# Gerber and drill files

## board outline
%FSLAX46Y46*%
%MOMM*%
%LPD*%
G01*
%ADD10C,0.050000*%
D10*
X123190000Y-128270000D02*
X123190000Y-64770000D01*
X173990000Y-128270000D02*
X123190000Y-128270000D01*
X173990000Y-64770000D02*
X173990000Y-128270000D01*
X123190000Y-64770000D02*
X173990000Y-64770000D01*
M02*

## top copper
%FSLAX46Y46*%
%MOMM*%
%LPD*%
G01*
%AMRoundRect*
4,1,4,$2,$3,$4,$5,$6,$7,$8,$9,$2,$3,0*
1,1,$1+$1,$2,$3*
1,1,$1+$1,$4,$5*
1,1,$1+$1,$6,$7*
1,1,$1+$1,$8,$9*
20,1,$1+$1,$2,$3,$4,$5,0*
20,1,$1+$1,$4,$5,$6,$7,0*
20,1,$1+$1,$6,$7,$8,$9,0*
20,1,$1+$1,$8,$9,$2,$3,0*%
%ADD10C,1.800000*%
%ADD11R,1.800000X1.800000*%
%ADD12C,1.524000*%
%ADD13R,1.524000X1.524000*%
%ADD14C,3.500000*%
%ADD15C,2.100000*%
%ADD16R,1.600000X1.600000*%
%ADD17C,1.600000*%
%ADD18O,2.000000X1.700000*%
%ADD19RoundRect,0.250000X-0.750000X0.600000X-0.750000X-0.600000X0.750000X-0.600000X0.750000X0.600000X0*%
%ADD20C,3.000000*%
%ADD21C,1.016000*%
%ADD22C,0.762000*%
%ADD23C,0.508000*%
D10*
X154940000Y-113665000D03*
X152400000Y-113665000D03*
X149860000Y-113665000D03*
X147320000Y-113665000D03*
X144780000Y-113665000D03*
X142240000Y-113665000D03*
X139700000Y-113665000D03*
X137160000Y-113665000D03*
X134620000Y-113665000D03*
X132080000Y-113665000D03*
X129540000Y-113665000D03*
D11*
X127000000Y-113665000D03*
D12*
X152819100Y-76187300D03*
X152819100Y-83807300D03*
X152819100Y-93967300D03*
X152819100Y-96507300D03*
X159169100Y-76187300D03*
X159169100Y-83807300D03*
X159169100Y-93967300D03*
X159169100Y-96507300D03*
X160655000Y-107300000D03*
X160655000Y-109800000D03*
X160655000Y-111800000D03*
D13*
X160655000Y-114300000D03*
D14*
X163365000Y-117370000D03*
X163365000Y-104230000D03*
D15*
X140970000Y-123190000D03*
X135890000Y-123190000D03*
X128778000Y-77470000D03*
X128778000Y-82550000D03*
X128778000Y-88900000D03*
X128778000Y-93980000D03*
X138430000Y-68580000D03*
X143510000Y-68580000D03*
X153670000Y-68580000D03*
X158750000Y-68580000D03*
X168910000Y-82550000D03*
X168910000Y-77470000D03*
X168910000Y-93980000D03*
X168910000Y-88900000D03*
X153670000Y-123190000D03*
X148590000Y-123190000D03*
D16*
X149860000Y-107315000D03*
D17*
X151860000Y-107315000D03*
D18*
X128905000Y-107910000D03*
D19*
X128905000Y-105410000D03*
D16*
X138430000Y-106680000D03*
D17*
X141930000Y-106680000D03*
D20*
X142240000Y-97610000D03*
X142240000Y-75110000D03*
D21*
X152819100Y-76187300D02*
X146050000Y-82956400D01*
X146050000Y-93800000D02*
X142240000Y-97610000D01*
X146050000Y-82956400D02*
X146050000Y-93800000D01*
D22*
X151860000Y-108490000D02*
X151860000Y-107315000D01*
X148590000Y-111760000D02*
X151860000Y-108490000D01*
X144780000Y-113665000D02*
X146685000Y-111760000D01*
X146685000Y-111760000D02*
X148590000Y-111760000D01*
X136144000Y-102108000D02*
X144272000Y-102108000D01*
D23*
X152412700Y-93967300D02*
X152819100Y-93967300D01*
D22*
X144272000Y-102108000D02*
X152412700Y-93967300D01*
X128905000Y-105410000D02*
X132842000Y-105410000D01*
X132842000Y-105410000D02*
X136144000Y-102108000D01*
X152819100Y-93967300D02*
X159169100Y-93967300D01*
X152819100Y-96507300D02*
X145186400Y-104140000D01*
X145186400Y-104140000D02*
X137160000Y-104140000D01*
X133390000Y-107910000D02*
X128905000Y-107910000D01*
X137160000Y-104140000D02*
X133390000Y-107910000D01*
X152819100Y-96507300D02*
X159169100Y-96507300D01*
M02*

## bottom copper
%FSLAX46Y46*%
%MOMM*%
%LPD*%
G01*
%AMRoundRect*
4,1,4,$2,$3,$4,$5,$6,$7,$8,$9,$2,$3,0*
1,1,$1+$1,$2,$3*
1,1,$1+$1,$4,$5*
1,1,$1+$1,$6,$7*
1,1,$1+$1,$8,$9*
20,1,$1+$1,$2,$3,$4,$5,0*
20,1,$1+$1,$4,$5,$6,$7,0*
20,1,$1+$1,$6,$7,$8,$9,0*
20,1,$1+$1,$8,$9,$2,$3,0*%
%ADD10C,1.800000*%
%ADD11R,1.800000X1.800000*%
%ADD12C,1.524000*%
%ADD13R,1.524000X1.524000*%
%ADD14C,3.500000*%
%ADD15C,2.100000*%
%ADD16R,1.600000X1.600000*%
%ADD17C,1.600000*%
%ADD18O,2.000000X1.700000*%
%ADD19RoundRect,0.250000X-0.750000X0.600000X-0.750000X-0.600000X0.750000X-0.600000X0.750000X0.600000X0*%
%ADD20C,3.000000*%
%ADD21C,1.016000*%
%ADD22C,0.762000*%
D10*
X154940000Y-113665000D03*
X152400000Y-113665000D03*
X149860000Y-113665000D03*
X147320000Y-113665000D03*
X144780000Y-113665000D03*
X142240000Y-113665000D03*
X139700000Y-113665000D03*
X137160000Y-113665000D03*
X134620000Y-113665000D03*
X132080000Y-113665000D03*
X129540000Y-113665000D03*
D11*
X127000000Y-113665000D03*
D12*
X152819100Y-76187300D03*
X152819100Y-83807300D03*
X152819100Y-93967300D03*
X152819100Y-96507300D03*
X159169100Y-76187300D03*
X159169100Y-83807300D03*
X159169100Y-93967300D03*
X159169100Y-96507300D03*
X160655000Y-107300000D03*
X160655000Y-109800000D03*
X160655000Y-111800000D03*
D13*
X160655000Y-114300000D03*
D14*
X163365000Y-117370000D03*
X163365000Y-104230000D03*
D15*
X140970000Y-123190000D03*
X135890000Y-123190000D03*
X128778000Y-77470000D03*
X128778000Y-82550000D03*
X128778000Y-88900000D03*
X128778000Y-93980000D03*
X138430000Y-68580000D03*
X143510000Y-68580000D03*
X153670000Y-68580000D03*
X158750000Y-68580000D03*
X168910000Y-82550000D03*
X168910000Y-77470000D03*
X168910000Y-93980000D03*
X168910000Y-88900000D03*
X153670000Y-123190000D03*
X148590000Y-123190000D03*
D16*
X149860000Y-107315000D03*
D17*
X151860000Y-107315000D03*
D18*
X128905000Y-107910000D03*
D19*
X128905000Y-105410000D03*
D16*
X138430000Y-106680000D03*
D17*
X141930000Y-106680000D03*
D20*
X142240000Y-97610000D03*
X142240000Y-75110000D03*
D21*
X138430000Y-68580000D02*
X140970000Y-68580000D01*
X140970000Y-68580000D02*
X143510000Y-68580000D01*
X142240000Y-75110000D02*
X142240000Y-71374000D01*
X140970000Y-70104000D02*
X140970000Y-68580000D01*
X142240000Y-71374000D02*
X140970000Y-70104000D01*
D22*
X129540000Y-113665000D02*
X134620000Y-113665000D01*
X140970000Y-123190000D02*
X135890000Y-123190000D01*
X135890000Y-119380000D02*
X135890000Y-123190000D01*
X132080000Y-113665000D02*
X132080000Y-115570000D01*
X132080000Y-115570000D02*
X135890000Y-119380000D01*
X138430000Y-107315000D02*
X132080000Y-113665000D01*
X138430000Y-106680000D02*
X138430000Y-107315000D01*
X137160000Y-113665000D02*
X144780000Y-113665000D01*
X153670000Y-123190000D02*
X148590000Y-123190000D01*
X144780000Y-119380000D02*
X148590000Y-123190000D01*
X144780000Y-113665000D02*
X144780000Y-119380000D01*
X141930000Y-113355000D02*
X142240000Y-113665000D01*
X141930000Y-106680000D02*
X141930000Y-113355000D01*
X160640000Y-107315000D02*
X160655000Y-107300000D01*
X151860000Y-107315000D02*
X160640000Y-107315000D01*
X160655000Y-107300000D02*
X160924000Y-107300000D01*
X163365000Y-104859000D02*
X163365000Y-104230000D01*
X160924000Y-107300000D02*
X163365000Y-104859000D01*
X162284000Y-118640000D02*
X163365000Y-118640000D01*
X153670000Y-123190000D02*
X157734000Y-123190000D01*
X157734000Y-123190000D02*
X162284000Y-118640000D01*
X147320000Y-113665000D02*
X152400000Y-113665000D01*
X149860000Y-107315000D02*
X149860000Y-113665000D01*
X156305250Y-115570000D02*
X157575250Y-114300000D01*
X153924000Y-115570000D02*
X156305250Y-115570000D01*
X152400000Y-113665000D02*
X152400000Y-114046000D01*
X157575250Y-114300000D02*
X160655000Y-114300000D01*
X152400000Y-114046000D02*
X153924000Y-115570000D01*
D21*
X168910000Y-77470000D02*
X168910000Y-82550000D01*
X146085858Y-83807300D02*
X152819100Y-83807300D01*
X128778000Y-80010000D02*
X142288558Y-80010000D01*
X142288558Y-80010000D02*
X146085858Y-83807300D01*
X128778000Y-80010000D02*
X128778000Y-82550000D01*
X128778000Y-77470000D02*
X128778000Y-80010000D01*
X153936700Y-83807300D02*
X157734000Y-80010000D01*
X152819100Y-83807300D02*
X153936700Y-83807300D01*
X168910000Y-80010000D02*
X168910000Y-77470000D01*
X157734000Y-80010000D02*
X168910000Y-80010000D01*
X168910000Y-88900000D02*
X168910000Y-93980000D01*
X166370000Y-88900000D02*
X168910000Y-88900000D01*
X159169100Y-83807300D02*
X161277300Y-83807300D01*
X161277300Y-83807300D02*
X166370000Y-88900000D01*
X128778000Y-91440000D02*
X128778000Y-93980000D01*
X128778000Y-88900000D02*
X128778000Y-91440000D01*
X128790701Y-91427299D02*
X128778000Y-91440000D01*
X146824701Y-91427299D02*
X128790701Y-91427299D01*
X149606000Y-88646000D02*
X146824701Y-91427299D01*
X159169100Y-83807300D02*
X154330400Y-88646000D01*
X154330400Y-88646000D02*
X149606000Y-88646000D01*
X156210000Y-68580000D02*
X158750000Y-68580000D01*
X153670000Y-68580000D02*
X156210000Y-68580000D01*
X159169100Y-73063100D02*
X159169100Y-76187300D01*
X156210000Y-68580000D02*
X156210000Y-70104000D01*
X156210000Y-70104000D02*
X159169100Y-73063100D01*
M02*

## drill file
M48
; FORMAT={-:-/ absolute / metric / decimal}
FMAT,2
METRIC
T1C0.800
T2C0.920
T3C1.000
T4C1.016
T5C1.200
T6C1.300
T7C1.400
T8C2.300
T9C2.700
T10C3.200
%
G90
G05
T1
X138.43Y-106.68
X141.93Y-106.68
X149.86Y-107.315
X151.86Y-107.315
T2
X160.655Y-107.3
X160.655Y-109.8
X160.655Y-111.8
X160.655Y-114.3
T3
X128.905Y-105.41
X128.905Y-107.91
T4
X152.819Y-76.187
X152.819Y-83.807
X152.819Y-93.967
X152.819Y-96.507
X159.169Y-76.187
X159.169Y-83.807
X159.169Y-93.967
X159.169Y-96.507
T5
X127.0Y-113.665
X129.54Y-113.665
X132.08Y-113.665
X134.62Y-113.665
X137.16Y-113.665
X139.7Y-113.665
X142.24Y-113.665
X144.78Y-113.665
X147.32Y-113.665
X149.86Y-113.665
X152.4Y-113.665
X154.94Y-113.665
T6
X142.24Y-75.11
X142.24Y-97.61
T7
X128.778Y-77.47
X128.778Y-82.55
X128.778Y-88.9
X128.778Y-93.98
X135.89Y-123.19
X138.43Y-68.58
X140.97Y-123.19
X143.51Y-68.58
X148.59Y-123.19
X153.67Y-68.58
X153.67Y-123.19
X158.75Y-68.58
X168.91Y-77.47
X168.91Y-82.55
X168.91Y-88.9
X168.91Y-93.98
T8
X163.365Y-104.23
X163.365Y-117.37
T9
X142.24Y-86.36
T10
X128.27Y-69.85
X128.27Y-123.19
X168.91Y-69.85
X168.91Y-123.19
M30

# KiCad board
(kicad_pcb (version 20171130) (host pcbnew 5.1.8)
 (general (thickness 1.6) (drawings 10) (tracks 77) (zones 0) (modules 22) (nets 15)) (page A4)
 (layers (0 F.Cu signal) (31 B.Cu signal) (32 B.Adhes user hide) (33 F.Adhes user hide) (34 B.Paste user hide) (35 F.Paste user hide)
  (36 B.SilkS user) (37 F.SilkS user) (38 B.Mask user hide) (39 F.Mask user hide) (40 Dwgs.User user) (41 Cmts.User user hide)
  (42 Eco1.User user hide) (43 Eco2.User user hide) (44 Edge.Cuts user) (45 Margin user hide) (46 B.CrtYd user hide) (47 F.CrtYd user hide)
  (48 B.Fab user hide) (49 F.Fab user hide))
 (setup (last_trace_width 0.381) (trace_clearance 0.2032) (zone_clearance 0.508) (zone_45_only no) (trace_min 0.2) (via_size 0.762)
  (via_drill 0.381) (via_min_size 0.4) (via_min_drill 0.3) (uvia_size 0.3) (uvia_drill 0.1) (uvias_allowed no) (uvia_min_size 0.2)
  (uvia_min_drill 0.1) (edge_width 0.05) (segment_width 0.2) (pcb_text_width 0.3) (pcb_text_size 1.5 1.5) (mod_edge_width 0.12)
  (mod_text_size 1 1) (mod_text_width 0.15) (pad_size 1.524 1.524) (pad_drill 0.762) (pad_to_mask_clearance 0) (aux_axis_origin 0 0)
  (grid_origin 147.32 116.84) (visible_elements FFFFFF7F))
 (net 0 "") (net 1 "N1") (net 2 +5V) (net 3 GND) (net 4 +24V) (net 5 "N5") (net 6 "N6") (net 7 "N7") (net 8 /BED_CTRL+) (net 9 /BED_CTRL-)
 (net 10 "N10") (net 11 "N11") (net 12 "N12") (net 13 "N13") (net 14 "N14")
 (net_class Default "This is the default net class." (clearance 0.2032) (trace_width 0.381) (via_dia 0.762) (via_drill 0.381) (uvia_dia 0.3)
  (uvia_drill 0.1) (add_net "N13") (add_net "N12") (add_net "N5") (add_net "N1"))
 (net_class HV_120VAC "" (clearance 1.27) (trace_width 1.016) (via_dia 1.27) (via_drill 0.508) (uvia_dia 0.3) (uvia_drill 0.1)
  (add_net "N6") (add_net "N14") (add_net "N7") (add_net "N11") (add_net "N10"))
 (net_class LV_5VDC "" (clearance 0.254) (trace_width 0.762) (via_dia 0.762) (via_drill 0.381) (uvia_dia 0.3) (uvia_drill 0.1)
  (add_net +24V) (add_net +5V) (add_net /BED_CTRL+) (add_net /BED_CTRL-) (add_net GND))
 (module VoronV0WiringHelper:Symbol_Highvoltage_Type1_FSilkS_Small (layer F.Cu) (at 131.064 71.628)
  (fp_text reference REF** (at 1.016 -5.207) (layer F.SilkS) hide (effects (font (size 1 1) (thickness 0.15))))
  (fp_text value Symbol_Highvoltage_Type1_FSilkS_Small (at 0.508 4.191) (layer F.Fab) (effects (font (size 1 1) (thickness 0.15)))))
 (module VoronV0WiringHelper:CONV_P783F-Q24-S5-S (layer F.Cu) (at 127 113.665)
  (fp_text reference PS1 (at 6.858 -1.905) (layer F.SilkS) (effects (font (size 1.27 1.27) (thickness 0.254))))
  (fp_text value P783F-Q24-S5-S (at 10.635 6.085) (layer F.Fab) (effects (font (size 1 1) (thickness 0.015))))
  (pad 12 thru_hole circle (at 27.94 0) (size 1.8 1.8) (drill 1.2) (layers *.Cu *.Mask) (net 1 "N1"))
  (pad 11 thru_hole circle (at 25.4 0) (size 1.8 1.8) (drill 1.2) (layers *.Cu *.Mask) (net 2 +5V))
  (pad 10 thru_hole circle (at 22.86 0) (size 1.8 1.8) (drill 1.2) (layers *.Cu *.Mask) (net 2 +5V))
  (pad 9 thru_hole circle (at 20.32 0) (size 1.8 1.8) (drill 1.2) (layers *.Cu *.Mask) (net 2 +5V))
  (pad 8 thru_hole circle (at 17.78 0) (size 1.8 1.8) (drill 1.2) (layers *.Cu *.Mask) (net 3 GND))
  (pad 7 thru_hole circle (at 15.24 0) (size 1.8 1.8) (drill 1.2) (layers *.Cu *.Mask) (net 3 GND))
  (pad 6 thru_hole circle (at 12.7 0) (size 1.8 1.8) (drill 1.2) (layers *.Cu *.Mask) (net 3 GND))
  (pad 5 thru_hole circle (at 10.16 0) (size 1.8 1.8) (drill 1.2) (layers *.Cu *.Mask) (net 3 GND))
  (pad 4 thru_hole circle (at 7.62 0) (size 1.8 1.8) (drill 1.2) (layers *.Cu *.Mask) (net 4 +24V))
  (pad 3 thru_hole circle (at 5.08 0) (size 1.8 1.8) (drill 1.2) (layers *.Cu *.Mask) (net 4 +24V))
  (pad 2 thru_hole circle (at 2.54 0) (size 1.8 1.8) (drill 1.2) (layers *.Cu *.Mask) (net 4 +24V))
  (pad 1 thru_hole rect (at 0 0) (size 1.8 1.8) (drill 1.2) (layers *.Cu *.Mask) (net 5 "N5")))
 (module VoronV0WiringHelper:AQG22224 (layer F.Cu) (at 151.765 86.36 180)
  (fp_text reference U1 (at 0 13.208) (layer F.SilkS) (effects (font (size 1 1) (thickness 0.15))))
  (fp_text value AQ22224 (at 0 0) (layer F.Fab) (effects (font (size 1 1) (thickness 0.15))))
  (pad 4 thru_hole circle (at -1.0541 10.1727 180) (size 1.524 1.524) (drill 1.016) (layers *.Cu *.Mask) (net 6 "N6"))
  (pad 3 thru_hole circle (at -1.0541 2.5527 180) (size 1.524 1.524) (drill 1.016) (layers *.Cu *.Mask) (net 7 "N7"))
  (pad 2 thru_hole circle (at -1.0541 -7.6073 180) (size 1.524 1.524) (drill 1.016) (layers *.Cu *.Mask) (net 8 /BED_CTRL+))
  (pad 1 thru_hole circle (at -1.0541 -10.1473 180) (size 1.524 1.524) (drill 1.016) (layers *.Cu *.Mask) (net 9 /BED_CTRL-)))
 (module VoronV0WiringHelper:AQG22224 (layer F.Cu) (at 158.115 86.36 180)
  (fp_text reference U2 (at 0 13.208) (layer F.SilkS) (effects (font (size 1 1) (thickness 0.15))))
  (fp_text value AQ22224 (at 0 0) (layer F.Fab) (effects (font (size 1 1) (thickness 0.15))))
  (pad 4 thru_hole circle (at -1.0541 10.1727 180) (size 1.524 1.524) (drill 1.016) (layers *.Cu *.Mask) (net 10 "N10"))
  (pad 3 thru_hole circle (at -1.0541 2.5527 180) (size 1.524 1.524) (drill 1.016) (layers *.Cu *.Mask) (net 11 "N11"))
  (pad 2 thru_hole circle (at -1.0541 -7.6073 180) (size 1.524 1.524) (drill 1.016) (layers *.Cu *.Mask) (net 8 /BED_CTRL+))
  (pad 1 thru_hole circle (at -1.0541 -10.1473 180) (size 1.524 1.524) (drill 1.016) (layers *.Cu *.Mask) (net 9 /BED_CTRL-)))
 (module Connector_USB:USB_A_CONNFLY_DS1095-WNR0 (layer F.Cu) (at 160.655 114.3 90)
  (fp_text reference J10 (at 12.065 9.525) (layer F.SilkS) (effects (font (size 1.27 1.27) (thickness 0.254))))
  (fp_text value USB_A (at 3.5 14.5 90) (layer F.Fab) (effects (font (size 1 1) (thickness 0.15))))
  (pad 4 thru_hole circle (at 7 0 90) (size 1.524 1.524) (drill 0.92) (layers *.Cu *.Mask) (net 3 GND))
  (pad 3 thru_hole circle (at 4.5 0 90) (size 1.524 1.524) (drill 0.92) (layers *.Cu *.Mask) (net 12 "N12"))
  (pad 2 thru_hole circle (at 2.5 0 90) (size 1.524 1.524) (drill 0.92) (layers *.Cu *.Mask) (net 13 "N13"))
  (pad 1 thru_hole rect (at 0 0 90) (size 1.524 1.524) (drill 0.92) (layers *.Cu *.Mask) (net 2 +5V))
  (pad 5 thru_hole circle (at -3.07 2.71 90) (size 3.5 3.5) (drill 2.3) (layers *.Cu *.Mask) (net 3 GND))
  (pad 5 thru_hole circle (at 10.07 2.71 90) (size 3.5 3.5) (drill 2.3) (layers *.Cu *.Mask) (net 3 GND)))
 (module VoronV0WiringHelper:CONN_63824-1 (layer F.Cu) (at 138.43 123.19 180)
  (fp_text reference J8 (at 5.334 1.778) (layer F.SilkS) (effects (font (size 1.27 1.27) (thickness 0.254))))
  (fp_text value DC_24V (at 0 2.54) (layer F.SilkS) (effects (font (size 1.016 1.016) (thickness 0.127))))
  (pad 1 thru_hole circle (at -2.54 0 180) (size 2.1 2.1) (drill 1.4) (layers *.Cu *.Mask) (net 4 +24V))
  (pad 1 thru_hole circle (at 2.54 0 180) (size 2.1 2.1) (drill 1.4) (layers *.Cu *.Mask) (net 4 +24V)))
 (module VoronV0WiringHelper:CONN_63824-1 (layer F.Cu) (at 128.778 80.01 270)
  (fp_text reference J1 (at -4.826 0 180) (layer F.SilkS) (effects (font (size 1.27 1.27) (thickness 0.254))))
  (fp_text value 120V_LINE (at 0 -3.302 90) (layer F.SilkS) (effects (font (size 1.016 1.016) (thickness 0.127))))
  (pad 1 thru_hole circle (at -2.54 0 270) (size 2.1 2.1) (drill 1.4) (layers *.Cu *.Mask) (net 7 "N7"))
  (pad 1 thru_hole circle (at 2.54 0 270) (size 2.1 2.1) (drill 1.4) (layers *.Cu *.Mask) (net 7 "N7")))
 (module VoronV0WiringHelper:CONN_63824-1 (layer F.Cu) (at 128.778 91.44 270)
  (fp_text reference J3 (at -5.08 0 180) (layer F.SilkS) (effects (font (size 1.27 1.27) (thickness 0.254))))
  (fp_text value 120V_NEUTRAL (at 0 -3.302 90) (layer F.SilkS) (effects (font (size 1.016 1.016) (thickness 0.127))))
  (pad 1 thru_hole circle (at -2.54 0 270) (size 2.1 2.1) (drill 1.4) (layers *.Cu *.Mask) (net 11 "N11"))
  (pad 1 thru_hole circle (at 2.54 0 270) (size 2.1 2.1) (drill 1.4) (layers *.Cu *.Mask) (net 11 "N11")))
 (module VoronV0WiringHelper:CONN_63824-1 (layer F.Cu) (at 140.97 68.58)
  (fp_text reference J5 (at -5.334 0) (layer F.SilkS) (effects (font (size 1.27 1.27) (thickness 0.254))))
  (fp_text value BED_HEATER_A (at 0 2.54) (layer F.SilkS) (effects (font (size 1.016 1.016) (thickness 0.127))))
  (pad 1 thru_hole circle (at -2.54 0) (size 2.1 2.1) (drill 1.4) (layers *.Cu *.Mask) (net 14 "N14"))
  (pad 1 thru_hole circle (at 2.54 0) (size 2.1 2.1) (drill 1.4) (layers *.Cu *.Mask) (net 14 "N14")))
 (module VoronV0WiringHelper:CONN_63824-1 (layer F.Cu) (at 156.21 68.58)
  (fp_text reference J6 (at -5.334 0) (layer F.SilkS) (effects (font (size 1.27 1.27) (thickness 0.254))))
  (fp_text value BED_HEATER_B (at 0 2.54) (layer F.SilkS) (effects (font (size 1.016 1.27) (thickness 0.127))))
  (pad 1 thru_hole circle (at -2.54 0) (size 2.1 2.1) (drill 1.4) (layers *.Cu *.Mask) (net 10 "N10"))
  (pad 1 thru_hole circle (at 2.54 0) (size 2.1 2.1) (drill 1.4) (layers *.Cu *.Mask) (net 10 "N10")))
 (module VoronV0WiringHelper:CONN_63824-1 (layer F.Cu) (at 168.91 80.01 90)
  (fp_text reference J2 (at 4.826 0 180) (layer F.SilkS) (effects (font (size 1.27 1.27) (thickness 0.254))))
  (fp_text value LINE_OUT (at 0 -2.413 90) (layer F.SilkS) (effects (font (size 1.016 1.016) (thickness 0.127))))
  (pad 1 thru_hole circle (at -2.54 0 90) (size 2.1 2.1) (drill 1.4) (layers *.Cu *.Mask) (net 7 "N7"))
  (pad 1 thru_hole circle (at 2.54 0 90) (size 2.1 2.1) (drill 1.4) (layers *.Cu *.Mask) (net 7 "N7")))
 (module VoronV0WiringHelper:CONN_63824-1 (layer F.Cu) (at 168.91 91.44 90)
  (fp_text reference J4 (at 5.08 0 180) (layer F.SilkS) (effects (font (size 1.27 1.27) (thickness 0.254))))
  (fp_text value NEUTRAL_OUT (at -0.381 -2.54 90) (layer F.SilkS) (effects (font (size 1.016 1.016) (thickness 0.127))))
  (pad 1 thru_hole circle (at -2.54 0 90) (size 2.1 2.1) (drill 1.4) (layers *.Cu *.Mask) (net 11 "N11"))
  (pad 1 thru_hole circle (at 2.54 0 90) (size 2.1 2.1) (drill 1.4) (layers *.Cu *.Mask) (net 11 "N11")))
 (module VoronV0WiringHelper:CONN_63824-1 (layer F.Cu) (at 151.13 123.19 180)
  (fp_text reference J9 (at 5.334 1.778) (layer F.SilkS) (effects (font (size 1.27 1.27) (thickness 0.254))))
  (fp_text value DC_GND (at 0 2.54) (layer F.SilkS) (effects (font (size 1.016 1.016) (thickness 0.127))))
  (pad 1 thru_hole circle (at -2.54 0 180) (size 2.1 2.1) (drill 1.4) (layers *.Cu *.Mask) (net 3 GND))
  (pad 1 thru_hole circle (at 2.54 0 180) (size 2.1 2.1) (drill 1.4) (layers *.Cu *.Mask) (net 3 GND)))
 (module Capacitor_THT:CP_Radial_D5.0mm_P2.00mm (layer F.Cu) (at 149.86 107.315)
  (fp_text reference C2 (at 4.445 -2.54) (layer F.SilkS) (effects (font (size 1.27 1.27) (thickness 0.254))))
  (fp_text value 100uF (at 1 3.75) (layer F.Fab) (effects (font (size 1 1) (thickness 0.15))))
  (pad 1 thru_hole rect (at 0 0) (size 1.6 1.6) (drill 0.8) (layers *.Cu *.Mask) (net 2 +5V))
  (pad 2 thru_hole circle (at 2 0) (size 1.6 1.6) (drill 0.8) (layers *.Cu *.Mask) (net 3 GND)))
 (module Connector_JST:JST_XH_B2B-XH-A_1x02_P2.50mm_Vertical (layer F.Cu) (at 128.905 105.41 270)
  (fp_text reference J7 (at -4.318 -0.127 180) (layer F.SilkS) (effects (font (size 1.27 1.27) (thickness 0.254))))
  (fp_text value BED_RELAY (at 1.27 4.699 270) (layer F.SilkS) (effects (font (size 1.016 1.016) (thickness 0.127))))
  (pad 2 thru_hole oval (at 2.5 0 270) (size 1.7 2) (drill 1) (layers *.Cu *.Mask) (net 9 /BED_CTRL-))
  (pad 1 thru_hole roundrect (at 0 0 270) (size 1.7 2) (drill 1) (layers *.Cu *.Mask) (roundrect_rratio 0.1470588235294118)
   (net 8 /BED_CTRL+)))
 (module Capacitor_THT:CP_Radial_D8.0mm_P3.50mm (layer F.Cu) (at 138.43 106.68)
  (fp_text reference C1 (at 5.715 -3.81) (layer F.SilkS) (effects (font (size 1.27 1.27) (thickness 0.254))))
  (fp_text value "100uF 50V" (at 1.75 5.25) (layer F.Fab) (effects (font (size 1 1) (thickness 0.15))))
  (pad 1 thru_hole rect (at 0 0) (size 1.6 1.6) (drill 0.8) (layers *.Cu *.Mask) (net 4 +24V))
  (pad 2 thru_hole circle (at 3.5 0) (size 1.6 1.6) (drill 0.8) (layers *.Cu *.Mask) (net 3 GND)))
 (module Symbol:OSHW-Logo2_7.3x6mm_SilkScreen (layer F.Cu) (at 161.29 123.825)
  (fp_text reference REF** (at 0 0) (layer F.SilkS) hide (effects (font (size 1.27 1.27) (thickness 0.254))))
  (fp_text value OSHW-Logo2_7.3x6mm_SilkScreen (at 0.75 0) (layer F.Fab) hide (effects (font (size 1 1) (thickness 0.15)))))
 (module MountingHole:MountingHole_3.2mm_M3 (layer F.Cu) (at 168.91 123.19)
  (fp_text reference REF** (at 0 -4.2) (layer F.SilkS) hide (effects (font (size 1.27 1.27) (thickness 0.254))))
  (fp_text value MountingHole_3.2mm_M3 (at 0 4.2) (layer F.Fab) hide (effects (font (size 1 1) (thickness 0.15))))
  (pad 1 np_thru_hole circle (at 0 0) (size 3.2 3.2) (drill 3.2) (layers *.Cu *.Mask)))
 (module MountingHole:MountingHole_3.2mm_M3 (layer F.Cu) (at 168.91 69.85)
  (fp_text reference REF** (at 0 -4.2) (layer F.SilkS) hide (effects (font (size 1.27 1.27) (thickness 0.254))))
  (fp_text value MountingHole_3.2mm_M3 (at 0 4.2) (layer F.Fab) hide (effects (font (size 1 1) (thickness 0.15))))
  (pad 1 np_thru_hole circle (at 0 0) (size 3.2 3.2) (drill 3.2) (layers *.Cu *.Mask)))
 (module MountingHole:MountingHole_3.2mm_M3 (layer F.Cu) (at 128.27 69.85)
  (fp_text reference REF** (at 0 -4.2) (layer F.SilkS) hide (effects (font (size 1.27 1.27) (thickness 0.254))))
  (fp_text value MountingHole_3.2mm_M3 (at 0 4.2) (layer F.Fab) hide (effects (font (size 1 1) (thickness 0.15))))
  (pad 1 np_thru_hole circle (at 0 0) (size 3.2 3.2) (drill 3.2) (layers *.Cu *.Mask)))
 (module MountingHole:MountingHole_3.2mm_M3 (layer F.Cu) (at 128.27 123.19)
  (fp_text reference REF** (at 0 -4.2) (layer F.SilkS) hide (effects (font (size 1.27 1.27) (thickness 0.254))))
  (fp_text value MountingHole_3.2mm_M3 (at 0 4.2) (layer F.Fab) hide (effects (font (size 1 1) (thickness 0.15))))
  (pad 1 np_thru_hole circle (at 0 0) (size 3.2 3.2) (drill 3.2) (layers *.Cu *.Mask)))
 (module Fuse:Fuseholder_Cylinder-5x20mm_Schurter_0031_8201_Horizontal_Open (layer F.Cu) (at 142.24 97.61 90)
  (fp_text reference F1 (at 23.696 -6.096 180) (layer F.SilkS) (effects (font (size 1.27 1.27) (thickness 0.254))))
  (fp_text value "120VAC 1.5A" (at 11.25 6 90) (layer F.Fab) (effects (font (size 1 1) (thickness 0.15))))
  (pad 1 thru_hole circle (at 0 0 90) (size 3 3) (drill 1.3) (layers *.Cu *.Mask) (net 6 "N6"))
  (pad 2 thru_hole circle (at 22.5 0 90) (size 3 3) (drill 1.3) (layers *.Cu *.Mask) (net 14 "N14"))
  (pad "" np_thru_hole circle (at 11.25 0 90) (size 2.7 2.7) (drill 2.7) (layers *.Cu *.Mask)))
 (gr_line (start 123.19 128.27) (end 123.19 64.77) (layer Edge.Cuts) (width 0.05))
 (gr_line (start 173.99 128.27) (end 123.19 128.27) (layer Edge.Cuts) (width 0.05))
 (gr_line (start 173.99 64.77) (end 173.99 128.27) (layer Edge.Cuts) (width 0.05))
 (gr_line (start 123.19 64.77) (end 173.99 64.77) (layer Edge.Cuts) (width 0.05))
 (segment (start 138.43 68.58) (end 140.97 68.58) (width 1.016) (layer B.Cu) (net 14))
 (segment (start 140.97 68.58) (end 143.51 68.58) (width 1.016) (layer B.Cu) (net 14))
 (segment (start 142.24 75.11) (end 142.24 71.374) (width 1.016) (layer B.Cu) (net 14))
 (segment (start 140.97 70.104) (end 140.97 68.58) (width 1.016) (layer B.Cu) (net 14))
 (segment (start 142.24 71.374) (end 140.97 70.104) (width 1.016) (layer B.Cu) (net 14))
 (segment (start 152.8191 76.1873) (end 146.05 82.9564) (width 1.016) (layer F.Cu) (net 6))
 (segment (start 146.05 93.8) (end 142.24 97.61) (width 1.016) (layer F.Cu) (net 6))
 (segment (start 146.05 82.9564) (end 146.05 93.8) (width 1.016) (layer F.Cu) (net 6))
 (segment (start 129.54 113.665) (end 134.62 113.665) (width 0.762) (layer B.Cu) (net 4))
 (segment (start 140.97 123.19) (end 135.89 123.19) (width 0.762) (layer B.Cu) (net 4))
 (segment (start 135.89 119.38) (end 135.89 123.19) (width 0.762) (layer B.Cu) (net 4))
 (segment (start 132.08 113.665) (end 132.08 115.57) (width 0.762) (layer B.Cu) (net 4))
 (segment (start 132.08 115.57) (end 135.89 119.38) (width 0.762) (layer B.Cu) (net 4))
 (segment (start 138.43 107.315) (end 132.08 113.665) (width 0.762) (layer B.Cu) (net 4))
 (segment (start 138.43 106.68) (end 138.43 107.315) (width 0.762) (layer B.Cu) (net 4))
 (segment (start 137.16 113.665) (end 144.78 113.665) (width 0.762) (layer B.Cu) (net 3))
 (segment (start 153.67 123.19) (end 148.59 123.19) (width 0.762) (layer B.Cu) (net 3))
 (segment (start 144.78 119.38) (end 148.59 123.19) (width 0.762) (layer B.Cu) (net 3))
 (segment (start 144.78 113.665) (end 144.78 119.38) (width 0.762) (layer B.Cu) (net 3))
 (segment (start 141.93 113.355) (end 142.24 113.665) (width 0.762) (layer B.Cu) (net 3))
 (segment (start 141.93 106.68) (end 141.93 113.355) (width 0.762) (layer B.Cu) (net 3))
 (segment (start 151.86 108.49) (end 151.86 107.315) (width 0.762) (layer F.Cu) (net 3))
 (segment (start 148.59 111.76) (end 151.86 108.49) (width 0.762) (layer F.Cu) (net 3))
 (segment (start 144.78 113.665) (end 146.685 111.76) (width 0.762) (layer F.Cu) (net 3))
 (segment (start 146.685 111.76) (end 148.59 111.76) (width 0.762) (layer F.Cu) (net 3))
 (segment (start 160.64 107.315) (end 160.655 107.3) (width 0.762) (layer B.Cu) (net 3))
 (segment (start 151.86 107.315) (end 160.64 107.315) (width 0.762) (layer B.Cu) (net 3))
 (segment (start 160.655 107.3) (end 160.924 107.3) (width 0.762) (layer B.Cu) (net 3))
 (segment (start 163.365 104.859) (end 163.365 104.23) (width 0.762) (layer B.Cu) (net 3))
 (segment (start 160.924 107.3) (end 163.365 104.859) (width 0.762) (layer B.Cu) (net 3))
 (segment (start 162.284 118.64) (end 163.365 118.64) (width 0.762) (layer B.Cu) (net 3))
 (segment (start 153.67 123.19) (end 157.734 123.19) (width 0.762) (layer B.Cu) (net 3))
 (segment (start 157.734 123.19) (end 162.284 118.64) (width 0.762) (layer B.Cu) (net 3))
 (segment (start 147.32 113.665) (end 152.4 113.665) (width 0.762) (layer B.Cu) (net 2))
 (segment (start 149.86 107.315) (end 149.86 113.665) (width 0.762) (layer B.Cu) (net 2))
 (segment (start 156.30525 115.57) (end 157.57525 114.3) (width 0.762) (layer B.Cu) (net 2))
 (segment (start 153.924 115.57) (end 156.30525 115.57) (width 0.762) (layer B.Cu) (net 2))
 (segment (start 152.4 113.665) (end 152.4 114.046) (width 0.762) (layer B.Cu) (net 2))
 (segment (start 157.57525 114.3) (end 160.655 114.3) (width 0.762) (layer B.Cu) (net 2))
 (segment (start 152.4 114.046) (end 153.924 115.57) (width 0.762) (layer B.Cu) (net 2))
 (segment (start 136.144 102.108) (end 144.272 102.108) (width 0.762) (layer F.Cu) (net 8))
 (segment (start 152.4127 93.9673) (end 152.8191 93.9673) (width 0.508) (layer F.Cu) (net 8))
 (segment (start 144.272 102.108) (end 152.4127 93.9673) (width 0.762) (layer F.Cu) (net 8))
 (segment (start 128.905 105.41) (end 132.842 105.41) (width 0.762) (layer F.Cu) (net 8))
 (segment (start 132.842 105.41) (end 136.144 102.108) (width 0.762) (layer F.Cu) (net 8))
 (segment (start 152.8191 93.9673) (end 159.1691 93.9673) (width 0.762) (layer F.Cu) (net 8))
 (segment (start 152.8191 96.5073) (end 145.1864 104.14) (width 0.762) (layer F.Cu) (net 9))
 (segment (start 145.1864 104.14) (end 137.16 104.14) (width 0.762) (layer F.Cu) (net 9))
 (segment (start 133.39 107.91) (end 128.905 107.91) (width 0.762) (layer F.Cu) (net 9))
 (segment (start 137.16 104.14) (end 133.39 107.91) (width 0.762) (layer F.Cu) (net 9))
 (segment (start 152.8191 96.5073) (end 159.1691 96.5073) (width 0.762) (layer F.Cu) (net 9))
 (segment (start 168.91 77.47) (end 168.91 82.55) (width 1.016) (layer B.Cu) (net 7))
 (segment (start 146.085858 83.8073) (end 152.8191 83.8073) (width 1.016) (layer B.Cu) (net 7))
 (segment (start 128.778 80.01) (end 142.288558 80.01) (width 1.016) (layer B.Cu) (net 7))
 (segment (start 142.288558 80.01) (end 146.085858 83.8073) (width 1.016) (layer B.Cu) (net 7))
 (segment (start 128.778 80.01) (end 128.778 82.55) (width 1.016) (layer B.Cu) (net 7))
 (segment (start 128.778 77.47) (end 128.778 80.01) (width 1.016) (layer B.Cu) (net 7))
 (segment (start 153.9367 83.8073) (end 157.734 80.01) (width 1.016) (layer B.Cu) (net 7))
 (segment (start 152.8191 83.8073) (end 153.9367 83.8073) (width 1.016) (layer B.Cu) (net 7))
 (segment (start 168.91 80.01) (end 168.91 77.47) (width 1.016) (layer B.Cu) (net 7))
 (segment (start 157.734 80.01) (end 168.91 80.01) (width 1.016) (layer B.Cu) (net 7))
 (segment (start 168.91 88.9) (end 168.91 93.98) (width 1.016) (layer B.Cu) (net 11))
 (segment (start 166.37 88.9) (end 168.91 88.9) (width 1.016) (layer B.Cu) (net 11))
 (segment (start 159.1691 83.8073) (end 161.2773 83.8073) (width 1.016) (layer B.Cu) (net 11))
 (segment (start 161.2773 83.8073) (end 166.37 88.9) (width 1.016) (layer B.Cu) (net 11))
 (segment (start 128.778 91.44) (end 128.778 93.98) (width 1.016) (layer B.Cu) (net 11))
 (segment (start 128.778 88.9) (end 128.778 91.44) (width 1.016) (layer B.Cu) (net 11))
 (segment (start 128.790701 91.427299) (end 128.778 91.44) (width 1.016) (layer B.Cu) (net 11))
 (segment (start 146.824701 91.427299) (end 128.790701 91.427299) (width 1.016) (layer B.Cu) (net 11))
 (segment (start 149.606 88.646) (end 146.824701 91.427299) (width 1.016) (layer B.Cu) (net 11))
 (segment (start 159.1691 83.8073) (end 154.3304 88.646) (width 1.016) (layer B.Cu) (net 11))
 (segment (start 154.3304 88.646) (end 149.606 88.646) (width 1.016) (layer B.Cu) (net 11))
 (segment (start 156.21 68.58) (end 158.75 68.58) (width 1.016) (layer B.Cu) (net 10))
 (segment (start 153.67 68.58) (end 156.21 68.58) (width 1.016) (layer B.Cu) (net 10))
 (segment (start 159.1691 73.0631) (end 159.1691 76.1873) (width 1.016) (layer B.Cu) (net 10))
 (segment (start 156.21 68.58) (end 156.21 70.104) (width 1.016) (layer B.Cu) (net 10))
 (segment (start 156.21 70.104) (end 159.1691 73.0631) (width 1.016) (layer B.Cu) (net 10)))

